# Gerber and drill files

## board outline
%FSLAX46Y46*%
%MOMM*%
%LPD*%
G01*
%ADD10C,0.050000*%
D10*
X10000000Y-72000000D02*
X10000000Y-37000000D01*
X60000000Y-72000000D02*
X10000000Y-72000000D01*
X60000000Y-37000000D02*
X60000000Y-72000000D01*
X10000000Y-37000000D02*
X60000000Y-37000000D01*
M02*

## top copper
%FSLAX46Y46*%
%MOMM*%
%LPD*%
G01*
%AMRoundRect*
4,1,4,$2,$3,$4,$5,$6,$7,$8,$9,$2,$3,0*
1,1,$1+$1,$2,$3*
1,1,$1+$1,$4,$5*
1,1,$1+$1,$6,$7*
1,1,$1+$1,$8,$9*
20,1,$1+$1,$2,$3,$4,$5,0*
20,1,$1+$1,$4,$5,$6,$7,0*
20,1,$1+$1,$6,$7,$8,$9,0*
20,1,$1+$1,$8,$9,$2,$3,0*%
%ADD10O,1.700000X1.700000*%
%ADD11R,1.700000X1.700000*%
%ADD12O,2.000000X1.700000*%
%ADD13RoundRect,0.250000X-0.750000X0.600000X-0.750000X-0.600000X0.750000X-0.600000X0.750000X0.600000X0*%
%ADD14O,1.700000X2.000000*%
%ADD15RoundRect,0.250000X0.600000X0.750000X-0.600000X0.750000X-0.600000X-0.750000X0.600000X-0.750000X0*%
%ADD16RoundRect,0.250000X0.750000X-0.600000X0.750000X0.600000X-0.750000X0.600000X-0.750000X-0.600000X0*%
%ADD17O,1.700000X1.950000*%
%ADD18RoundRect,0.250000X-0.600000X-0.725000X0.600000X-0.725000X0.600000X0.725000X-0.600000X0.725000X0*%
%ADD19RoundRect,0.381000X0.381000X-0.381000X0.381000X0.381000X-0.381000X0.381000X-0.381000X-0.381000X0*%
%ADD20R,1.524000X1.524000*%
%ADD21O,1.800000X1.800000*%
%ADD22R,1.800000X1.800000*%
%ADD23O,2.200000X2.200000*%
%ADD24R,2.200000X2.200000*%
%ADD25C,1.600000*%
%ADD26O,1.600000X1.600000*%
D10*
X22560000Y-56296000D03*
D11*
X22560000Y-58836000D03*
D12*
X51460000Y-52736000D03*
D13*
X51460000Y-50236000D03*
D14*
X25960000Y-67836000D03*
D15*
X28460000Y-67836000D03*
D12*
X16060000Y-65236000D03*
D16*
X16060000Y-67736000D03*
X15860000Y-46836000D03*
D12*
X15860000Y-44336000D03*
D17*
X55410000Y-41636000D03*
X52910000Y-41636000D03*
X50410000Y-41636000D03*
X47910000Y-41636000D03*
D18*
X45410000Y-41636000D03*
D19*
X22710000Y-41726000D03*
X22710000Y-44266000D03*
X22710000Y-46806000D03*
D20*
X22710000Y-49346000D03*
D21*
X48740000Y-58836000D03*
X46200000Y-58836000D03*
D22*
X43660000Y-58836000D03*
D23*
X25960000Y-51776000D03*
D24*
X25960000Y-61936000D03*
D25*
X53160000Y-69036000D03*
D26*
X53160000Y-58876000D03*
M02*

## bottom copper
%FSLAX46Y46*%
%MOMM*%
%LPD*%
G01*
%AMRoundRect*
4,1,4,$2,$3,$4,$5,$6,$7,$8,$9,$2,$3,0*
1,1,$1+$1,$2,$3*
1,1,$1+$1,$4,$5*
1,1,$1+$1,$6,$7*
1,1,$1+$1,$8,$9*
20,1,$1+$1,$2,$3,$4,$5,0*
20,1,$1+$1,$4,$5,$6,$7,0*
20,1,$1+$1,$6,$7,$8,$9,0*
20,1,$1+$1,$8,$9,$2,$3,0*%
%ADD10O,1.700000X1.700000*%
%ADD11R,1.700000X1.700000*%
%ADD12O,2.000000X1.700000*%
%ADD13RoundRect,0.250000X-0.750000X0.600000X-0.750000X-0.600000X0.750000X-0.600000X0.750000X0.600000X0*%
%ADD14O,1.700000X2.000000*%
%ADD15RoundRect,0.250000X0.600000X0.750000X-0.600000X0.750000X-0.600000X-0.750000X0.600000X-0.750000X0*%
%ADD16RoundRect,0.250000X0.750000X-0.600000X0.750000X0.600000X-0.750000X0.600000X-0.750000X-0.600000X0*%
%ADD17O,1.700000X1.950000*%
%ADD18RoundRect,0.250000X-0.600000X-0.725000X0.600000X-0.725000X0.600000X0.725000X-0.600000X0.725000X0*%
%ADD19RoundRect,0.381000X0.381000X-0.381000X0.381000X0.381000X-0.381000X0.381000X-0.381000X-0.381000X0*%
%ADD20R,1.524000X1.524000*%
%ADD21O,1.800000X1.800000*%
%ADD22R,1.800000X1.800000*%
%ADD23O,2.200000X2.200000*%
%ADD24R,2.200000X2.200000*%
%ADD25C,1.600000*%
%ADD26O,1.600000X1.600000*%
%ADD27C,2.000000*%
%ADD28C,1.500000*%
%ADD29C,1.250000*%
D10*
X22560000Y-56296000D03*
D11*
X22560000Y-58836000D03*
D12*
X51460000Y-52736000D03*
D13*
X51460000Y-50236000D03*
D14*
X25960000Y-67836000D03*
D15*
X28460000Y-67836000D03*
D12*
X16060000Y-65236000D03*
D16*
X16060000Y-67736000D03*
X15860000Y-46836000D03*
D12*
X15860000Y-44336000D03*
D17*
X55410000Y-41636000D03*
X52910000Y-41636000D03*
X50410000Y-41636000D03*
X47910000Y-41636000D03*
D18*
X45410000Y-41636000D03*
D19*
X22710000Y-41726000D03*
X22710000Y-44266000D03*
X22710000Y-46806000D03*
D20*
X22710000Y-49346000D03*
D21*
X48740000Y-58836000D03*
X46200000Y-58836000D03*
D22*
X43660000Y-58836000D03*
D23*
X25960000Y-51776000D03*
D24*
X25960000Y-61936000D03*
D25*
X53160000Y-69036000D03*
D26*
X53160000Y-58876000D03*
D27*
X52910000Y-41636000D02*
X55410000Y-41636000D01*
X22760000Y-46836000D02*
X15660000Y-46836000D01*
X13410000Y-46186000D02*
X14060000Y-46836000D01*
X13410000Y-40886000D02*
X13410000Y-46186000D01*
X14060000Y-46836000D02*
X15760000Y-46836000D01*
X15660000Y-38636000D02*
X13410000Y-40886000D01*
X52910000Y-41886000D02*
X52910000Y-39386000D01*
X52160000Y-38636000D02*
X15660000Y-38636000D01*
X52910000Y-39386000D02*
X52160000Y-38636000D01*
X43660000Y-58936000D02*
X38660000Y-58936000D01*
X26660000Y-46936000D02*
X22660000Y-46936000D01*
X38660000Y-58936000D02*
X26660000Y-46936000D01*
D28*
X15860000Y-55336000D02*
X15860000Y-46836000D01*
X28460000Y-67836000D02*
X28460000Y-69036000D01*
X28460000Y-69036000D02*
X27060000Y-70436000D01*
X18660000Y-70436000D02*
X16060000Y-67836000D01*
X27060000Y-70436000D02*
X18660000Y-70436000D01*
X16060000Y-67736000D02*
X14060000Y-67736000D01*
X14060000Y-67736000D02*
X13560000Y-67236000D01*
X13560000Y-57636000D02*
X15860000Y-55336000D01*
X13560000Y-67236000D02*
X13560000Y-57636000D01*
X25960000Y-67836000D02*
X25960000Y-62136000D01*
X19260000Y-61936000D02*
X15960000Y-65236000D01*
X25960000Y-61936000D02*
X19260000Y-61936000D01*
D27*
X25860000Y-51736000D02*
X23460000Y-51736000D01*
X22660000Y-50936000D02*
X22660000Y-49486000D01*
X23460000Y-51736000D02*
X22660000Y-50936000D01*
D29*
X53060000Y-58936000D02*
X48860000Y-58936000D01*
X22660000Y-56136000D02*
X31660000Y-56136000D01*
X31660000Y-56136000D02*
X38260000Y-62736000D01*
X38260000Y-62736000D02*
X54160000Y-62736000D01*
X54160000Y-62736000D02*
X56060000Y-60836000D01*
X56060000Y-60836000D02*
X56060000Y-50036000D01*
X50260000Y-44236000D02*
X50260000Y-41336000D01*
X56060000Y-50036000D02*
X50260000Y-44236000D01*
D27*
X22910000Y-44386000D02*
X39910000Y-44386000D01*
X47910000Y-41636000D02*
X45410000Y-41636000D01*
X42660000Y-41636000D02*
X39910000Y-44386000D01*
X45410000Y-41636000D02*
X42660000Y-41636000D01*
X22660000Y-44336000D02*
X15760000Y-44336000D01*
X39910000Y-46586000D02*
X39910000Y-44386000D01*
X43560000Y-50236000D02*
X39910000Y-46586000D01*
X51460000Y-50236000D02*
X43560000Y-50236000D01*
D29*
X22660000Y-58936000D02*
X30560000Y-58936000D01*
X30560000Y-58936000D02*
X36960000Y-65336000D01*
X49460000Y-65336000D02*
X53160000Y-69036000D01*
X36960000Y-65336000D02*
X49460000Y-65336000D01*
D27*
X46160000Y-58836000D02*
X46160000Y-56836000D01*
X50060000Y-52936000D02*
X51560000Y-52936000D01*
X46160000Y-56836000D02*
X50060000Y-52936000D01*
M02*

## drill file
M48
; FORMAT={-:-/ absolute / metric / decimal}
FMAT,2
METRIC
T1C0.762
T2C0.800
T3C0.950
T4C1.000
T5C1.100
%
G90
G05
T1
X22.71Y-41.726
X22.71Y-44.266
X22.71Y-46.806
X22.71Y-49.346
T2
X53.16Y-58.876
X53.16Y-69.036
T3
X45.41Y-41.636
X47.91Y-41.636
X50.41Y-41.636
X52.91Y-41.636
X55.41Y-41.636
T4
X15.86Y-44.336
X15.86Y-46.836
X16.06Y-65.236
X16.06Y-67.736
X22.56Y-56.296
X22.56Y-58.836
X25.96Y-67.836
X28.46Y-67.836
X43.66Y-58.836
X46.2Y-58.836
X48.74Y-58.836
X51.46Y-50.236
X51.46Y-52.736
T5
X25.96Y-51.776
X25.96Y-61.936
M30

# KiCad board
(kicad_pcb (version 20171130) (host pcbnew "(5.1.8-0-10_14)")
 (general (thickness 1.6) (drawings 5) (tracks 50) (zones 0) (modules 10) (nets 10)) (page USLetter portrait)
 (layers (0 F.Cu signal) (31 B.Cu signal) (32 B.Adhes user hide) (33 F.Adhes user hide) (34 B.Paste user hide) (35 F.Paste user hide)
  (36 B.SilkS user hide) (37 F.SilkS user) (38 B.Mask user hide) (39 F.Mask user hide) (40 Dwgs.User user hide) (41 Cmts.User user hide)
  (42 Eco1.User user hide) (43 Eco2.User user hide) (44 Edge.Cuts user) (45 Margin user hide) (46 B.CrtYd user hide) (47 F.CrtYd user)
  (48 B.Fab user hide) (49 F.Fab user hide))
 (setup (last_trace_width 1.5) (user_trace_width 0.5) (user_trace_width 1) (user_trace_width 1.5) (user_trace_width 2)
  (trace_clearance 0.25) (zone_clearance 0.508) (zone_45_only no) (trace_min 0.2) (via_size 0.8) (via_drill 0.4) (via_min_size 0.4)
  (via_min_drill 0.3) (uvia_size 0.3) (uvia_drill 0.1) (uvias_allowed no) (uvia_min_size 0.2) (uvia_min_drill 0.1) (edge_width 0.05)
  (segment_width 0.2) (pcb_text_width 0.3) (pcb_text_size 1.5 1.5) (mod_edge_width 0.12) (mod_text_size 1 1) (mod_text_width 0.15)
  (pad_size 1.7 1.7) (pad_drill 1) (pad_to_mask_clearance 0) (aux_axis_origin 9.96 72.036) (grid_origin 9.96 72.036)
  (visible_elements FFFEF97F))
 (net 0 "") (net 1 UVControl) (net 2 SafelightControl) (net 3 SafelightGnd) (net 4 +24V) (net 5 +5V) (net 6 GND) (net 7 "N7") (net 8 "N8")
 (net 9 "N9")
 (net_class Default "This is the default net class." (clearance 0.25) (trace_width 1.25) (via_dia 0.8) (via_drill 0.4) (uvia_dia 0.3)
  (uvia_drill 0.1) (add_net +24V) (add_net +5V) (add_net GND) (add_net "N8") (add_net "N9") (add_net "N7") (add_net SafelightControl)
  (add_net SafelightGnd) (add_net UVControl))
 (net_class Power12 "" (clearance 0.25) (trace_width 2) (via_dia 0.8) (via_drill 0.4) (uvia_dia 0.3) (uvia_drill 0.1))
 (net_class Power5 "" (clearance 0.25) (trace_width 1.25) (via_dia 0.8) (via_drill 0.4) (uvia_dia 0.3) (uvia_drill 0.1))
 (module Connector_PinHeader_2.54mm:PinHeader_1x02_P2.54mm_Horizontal (layer F.Cu) (at 22.56 58.836 180)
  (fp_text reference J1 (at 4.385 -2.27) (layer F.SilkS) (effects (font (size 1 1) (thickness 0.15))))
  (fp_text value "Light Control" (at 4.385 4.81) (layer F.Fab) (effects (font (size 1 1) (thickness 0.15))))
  (pad 2 thru_hole oval (at 0 2.54 180) (size 1.7 1.7) (drill 1) (layers *.Cu *.Mask) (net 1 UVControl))
  (pad 1 thru_hole rect (at 0 0 180) (size 1.7 1.7) (drill 1) (layers *.Cu *.Mask) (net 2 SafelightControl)))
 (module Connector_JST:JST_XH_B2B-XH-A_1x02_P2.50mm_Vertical (layer F.Cu) (at 51.46 50.236 270)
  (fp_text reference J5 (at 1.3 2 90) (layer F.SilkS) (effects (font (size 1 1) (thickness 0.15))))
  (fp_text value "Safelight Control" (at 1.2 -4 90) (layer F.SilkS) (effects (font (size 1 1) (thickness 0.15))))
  (pad 2 thru_hole oval (at 2.5 0 270) (size 1.7 2) (drill 1) (layers *.Cu *.Mask) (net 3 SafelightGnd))
  (pad 1 thru_hole roundrect (at 0 0 270) (size 1.7 2) (drill 1) (layers *.Cu *.Mask) (roundrect_rratio 0.1470588235294118) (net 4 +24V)))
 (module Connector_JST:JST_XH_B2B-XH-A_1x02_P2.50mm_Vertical (layer F.Cu) (at 28.46 67.836 180)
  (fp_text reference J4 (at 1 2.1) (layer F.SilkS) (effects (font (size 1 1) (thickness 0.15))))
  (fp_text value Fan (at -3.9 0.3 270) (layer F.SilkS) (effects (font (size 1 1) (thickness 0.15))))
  (pad 2 thru_hole oval (at 2.5 0 180) (size 1.7 2) (drill 1) (layers *.Cu *.Mask) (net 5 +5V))
  (pad 1 thru_hole roundrect (at 0 0 180) (size 1.7 2) (drill 1) (layers *.Cu *.Mask) (roundrect_rratio 0.1470588235294118) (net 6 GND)))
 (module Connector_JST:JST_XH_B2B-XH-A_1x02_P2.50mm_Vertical (layer F.Cu) (at 16.06 67.736 90)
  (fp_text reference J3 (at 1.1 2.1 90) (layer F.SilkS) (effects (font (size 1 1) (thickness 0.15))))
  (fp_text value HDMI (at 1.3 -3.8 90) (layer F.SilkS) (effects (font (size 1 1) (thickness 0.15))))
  (pad 2 thru_hole oval (at 2.5 0 90) (size 1.7 2) (drill 1) (layers *.Cu *.Mask) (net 5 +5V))
  (pad 1 thru_hole roundrect (at 0 0 90) (size 1.7 2) (drill 1) (layers *.Cu *.Mask) (roundrect_rratio 0.1470588235294118) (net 6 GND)))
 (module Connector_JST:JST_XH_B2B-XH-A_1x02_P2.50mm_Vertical (layer F.Cu) (at 15.86 46.836 90)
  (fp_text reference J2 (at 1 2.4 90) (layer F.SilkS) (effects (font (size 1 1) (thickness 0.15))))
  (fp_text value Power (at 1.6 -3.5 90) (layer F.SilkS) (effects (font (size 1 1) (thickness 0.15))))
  (pad 1 thru_hole roundrect (at 0 0 90) (size 1.7 2) (drill 1) (layers *.Cu *.Mask) (roundrect_rratio 0.1470588235294118) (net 6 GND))
  (pad 2 thru_hole oval (at 2.5 0 90) (size 1.7 2) (drill 1) (layers *.Cu *.Mask) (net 4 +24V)))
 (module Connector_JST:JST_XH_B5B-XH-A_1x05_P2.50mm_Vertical (layer F.Cu) (at 45.41 41.636)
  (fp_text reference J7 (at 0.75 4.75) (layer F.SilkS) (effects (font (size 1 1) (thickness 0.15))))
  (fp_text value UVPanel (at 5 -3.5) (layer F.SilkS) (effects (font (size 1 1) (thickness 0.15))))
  (pad 5 thru_hole oval (at 10 0) (size 1.7 1.95) (drill 0.95) (layers *.Cu *.Mask) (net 6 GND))
  (pad 4 thru_hole oval (at 7.5 0) (size 1.7 1.95) (drill 0.95) (layers *.Cu *.Mask) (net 6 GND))
  (pad 3 thru_hole oval (at 5 0) (size 1.7 1.95) (drill 0.95) (layers *.Cu *.Mask) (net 1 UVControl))
  (pad 2 thru_hole oval (at 2.5 0) (size 1.7 1.95) (drill 0.95) (layers *.Cu *.Mask) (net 4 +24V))
  (pad 1 thru_hole roundrect (at 0 0) (size 1.7 1.95) (drill 0.95) (layers *.Cu *.Mask) (roundrect_rratio 0.1470588235294118) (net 4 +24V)))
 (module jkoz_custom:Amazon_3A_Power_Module (layer F.Cu) (at 30.66 45.636 90)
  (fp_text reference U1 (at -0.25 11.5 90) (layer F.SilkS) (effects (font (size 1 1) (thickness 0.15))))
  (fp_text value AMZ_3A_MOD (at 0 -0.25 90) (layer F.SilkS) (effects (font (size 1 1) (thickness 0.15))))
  (pad 4 thru_hole roundrect (at 3.91 -7.95 90) (size 1.524 1.524) (drill 0.762) (layers *.Cu *.Mask) (roundrect_rratio 0.25) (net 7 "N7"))
  (pad 3 thru_hole roundrect (at 1.37 -7.95 90) (size 1.524 1.524) (drill 0.762) (layers *.Cu *.Mask) (roundrect_rratio 0.25) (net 4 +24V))
  (pad 2 thru_hole roundrect (at -1.17 -7.95 90) (size 1.524 1.524) (drill 0.762) (layers *.Cu *.Mask) (roundrect_rratio 0.25) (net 6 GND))
  (pad 1 thru_hole rect (at -3.71 -7.95 90) (size 1.524 1.524) (drill 0.762) (layers *.Cu *.Mask) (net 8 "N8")))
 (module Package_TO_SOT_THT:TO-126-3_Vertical (layer F.Cu) (at 43.66 58.836)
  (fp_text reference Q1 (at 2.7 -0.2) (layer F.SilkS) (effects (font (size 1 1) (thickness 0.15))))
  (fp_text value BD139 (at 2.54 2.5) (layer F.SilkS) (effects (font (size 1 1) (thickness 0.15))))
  (pad 3 thru_hole oval (at 5.08 0) (size 1.8 1.8) (drill 1) (layers *.Cu *.Mask) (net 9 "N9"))
  (pad 2 thru_hole oval (at 2.54 0) (size 1.8 1.8) (drill 1) (layers *.Cu *.Mask) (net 3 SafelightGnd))
  (pad 1 thru_hole rect (at 0 0) (size 1.8 1.8) (drill 1) (layers *.Cu *.Mask) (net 6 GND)))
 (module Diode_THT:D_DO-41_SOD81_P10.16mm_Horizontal (layer F.Cu) (at 25.96 61.936 90)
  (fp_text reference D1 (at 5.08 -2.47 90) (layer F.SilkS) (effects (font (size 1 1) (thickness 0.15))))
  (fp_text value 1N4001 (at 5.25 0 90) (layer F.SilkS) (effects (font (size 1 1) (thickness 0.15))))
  (pad 2 thru_hole oval (at 10.16 0 90) (size 2.2 2.2) (drill 1.1) (layers *.Cu *.Mask) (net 8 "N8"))
  (pad 1 thru_hole rect (at 0 0 90) (size 2.2 2.2) (drill 1.1) (layers *.Cu *.Mask) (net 5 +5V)))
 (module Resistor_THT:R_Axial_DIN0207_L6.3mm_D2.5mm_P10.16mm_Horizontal (layer F.Cu) (at 53.16 69.036 90)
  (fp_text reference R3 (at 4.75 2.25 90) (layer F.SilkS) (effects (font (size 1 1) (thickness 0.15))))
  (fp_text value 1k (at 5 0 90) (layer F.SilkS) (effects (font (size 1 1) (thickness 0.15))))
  (pad 1 thru_hole circle (at 0 0 90) (size 1.6 1.6) (drill 0.8) (layers *.Cu *.Mask) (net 2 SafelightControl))
  (pad 2 thru_hole oval (at 10.16 0 90) (size 1.6 1.6) (drill 0.8) (layers *.Cu *.Mask) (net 9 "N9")))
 (gr_line (start 10 72) (end 10 37) (layer Edge.Cuts) (width 0.05))
 (gr_line (start 60 72) (end 10 72) (layer Edge.Cuts) (width 0.05))
 (gr_line (start 60 37) (end 60 72) (layer Edge.Cuts) (width 0.05))
 (gr_line (start 10 37) (end 60 37) (layer Edge.Cuts) (width 0.05))
 (segment (start 52.91 41.636) (end 55.41 41.636) (width 2) (layer B.Cu) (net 6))
 (segment (start 22.76 46.836) (end 15.66 46.836) (width 2) (layer B.Cu) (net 6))
 (segment (start 13.41 46.186) (end 14.06 46.836) (width 2) (layer B.Cu) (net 6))
 (segment (start 13.41 40.886) (end 13.41 46.186) (width 2) (layer B.Cu) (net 6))
 (segment (start 14.06 46.836) (end 15.76 46.836) (width 2) (layer B.Cu) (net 6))
 (segment (start 15.66 38.636) (end 13.41 40.886) (width 2) (layer B.Cu) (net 6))
 (segment (start 52.91 41.886) (end 52.91 39.386) (width 2) (layer B.Cu) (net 6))
 (segment (start 52.16 38.636) (end 15.66 38.636) (width 2) (layer B.Cu) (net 6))
 (segment (start 52.91 39.386) (end 52.16 38.636) (width 2) (layer B.Cu) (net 6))
 (segment (start 43.66 58.936) (end 38.66 58.936) (width 2) (layer B.Cu) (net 6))
 (segment (start 26.66 46.936) (end 22.66 46.936) (width 2) (layer B.Cu) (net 6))
 (segment (start 38.66 58.936) (end 26.66 46.936) (width 2) (layer B.Cu) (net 6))
 (segment (start 15.86 55.336) (end 15.86 46.836) (width 1.5) (layer B.Cu) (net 6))
 (segment (start 28.46 67.836) (end 28.46 69.036) (width 1.5) (layer B.Cu) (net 6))
 (segment (start 28.46 69.036) (end 27.06 70.436) (width 1.5) (layer B.Cu) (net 6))
 (segment (start 18.66 70.436) (end 16.06 67.836) (width 1.5) (layer B.Cu) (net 6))
 (segment (start 27.06 70.436) (end 18.66 70.436) (width 1.5) (layer B.Cu) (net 6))
 (segment (start 16.06 67.736) (end 14.06 67.736) (width 1.5) (layer B.Cu) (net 6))
 (segment (start 14.06 67.736) (end 13.56 67.236) (width 1.5) (layer B.Cu) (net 6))
 (segment (start 13.56 57.636) (end 15.86 55.336) (width 1.5) (layer B.Cu) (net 6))
 (segment (start 13.56 67.236) (end 13.56 57.636) (width 1.5) (layer B.Cu) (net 6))
 (segment (start 25.96 67.836) (end 25.96 62.136) (width 1.5) (layer B.Cu) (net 5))
 (segment (start 19.26 61.936) (end 15.96 65.236) (width 1.5) (layer B.Cu) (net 5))
 (segment (start 25.96 61.936) (end 19.26 61.936) (width 1.5) (layer B.Cu) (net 5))
 (segment (start 25.86 51.736) (end 23.46 51.736) (width 2) (layer B.Cu) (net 8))
 (segment (start 22.66 50.936) (end 22.66 49.486) (width 2) (layer B.Cu) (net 8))
 (segment (start 23.46 51.736) (end 22.66 50.936) (width 2) (layer B.Cu) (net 8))
 (segment (start 53.06 58.936) (end 48.86 58.936) (width 1.25) (layer B.Cu) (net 9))
 (segment (start 22.66 56.136) (end 31.66 56.136) (width 1.25) (layer B.Cu) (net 1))
 (segment (start 31.66 56.136) (end 38.26 62.736) (width 1.25) (layer B.Cu) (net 1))
 (segment (start 38.26 62.736) (end 54.16 62.736) (width 1.25) (layer B.Cu) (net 1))
 (segment (start 54.16 62.736) (end 56.06 60.836) (width 1.25) (layer B.Cu) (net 1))
 (segment (start 56.06 60.836) (end 56.06 50.036) (width 1.25) (layer B.Cu) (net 1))
 (segment (start 50.26 44.236) (end 50.26 41.336) (width 1.25) (layer B.Cu) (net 1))
 (segment (start 56.06 50.036) (end 50.26 44.236) (width 1.25) (layer B.Cu) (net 1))
 (segment (start 22.91 44.386) (end 39.91 44.386) (width 2) (layer B.Cu) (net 4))
 (segment (start 47.91 41.636) (end 45.41 41.636) (width 2) (layer B.Cu) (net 4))
 (segment (start 42.66 41.636) (end 39.91 44.386) (width 2) (layer B.Cu) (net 4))
 (segment (start 45.41 41.636) (end 42.66 41.636) (width 2) (layer B.Cu) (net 4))
 (segment (start 22.66 44.336) (end 15.76 44.336) (width 2) (layer B.Cu) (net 4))
 (segment (start 39.91 46.586) (end 39.91 44.386) (width 2) (layer B.Cu) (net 4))
 (segment (start 43.56 50.236) (end 39.91 46.586) (width 2) (layer B.Cu) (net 4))
 (segment (start 51.46 50.236) (end 43.56 50.236) (width 2) (layer B.Cu) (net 4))
 (segment (start 22.66 58.936) (end 30.56 58.936) (width 1.25) (layer B.Cu) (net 2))
 (segment (start 30.56 58.936) (end 36.96 65.336) (width 1.25) (layer B.Cu) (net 2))
 (segment (start 49.46 65.336) (end 53.16 69.036) (width 1.25) (layer B.Cu) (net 2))
 (segment (start 36.96 65.336) (end 49.46 65.336) (width 1.25) (layer B.Cu) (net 2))
 (segment (start 46.16 58.836) (end 46.16 56.836) (width 2) (layer B.Cu) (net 3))
 (segment (start 50.06 52.936) (end 51.56 52.936) (width 2) (layer B.Cu) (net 3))
 (segment (start 46.16 56.836) (end 50.06 52.936) (width 2) (layer B.Cu) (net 3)))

